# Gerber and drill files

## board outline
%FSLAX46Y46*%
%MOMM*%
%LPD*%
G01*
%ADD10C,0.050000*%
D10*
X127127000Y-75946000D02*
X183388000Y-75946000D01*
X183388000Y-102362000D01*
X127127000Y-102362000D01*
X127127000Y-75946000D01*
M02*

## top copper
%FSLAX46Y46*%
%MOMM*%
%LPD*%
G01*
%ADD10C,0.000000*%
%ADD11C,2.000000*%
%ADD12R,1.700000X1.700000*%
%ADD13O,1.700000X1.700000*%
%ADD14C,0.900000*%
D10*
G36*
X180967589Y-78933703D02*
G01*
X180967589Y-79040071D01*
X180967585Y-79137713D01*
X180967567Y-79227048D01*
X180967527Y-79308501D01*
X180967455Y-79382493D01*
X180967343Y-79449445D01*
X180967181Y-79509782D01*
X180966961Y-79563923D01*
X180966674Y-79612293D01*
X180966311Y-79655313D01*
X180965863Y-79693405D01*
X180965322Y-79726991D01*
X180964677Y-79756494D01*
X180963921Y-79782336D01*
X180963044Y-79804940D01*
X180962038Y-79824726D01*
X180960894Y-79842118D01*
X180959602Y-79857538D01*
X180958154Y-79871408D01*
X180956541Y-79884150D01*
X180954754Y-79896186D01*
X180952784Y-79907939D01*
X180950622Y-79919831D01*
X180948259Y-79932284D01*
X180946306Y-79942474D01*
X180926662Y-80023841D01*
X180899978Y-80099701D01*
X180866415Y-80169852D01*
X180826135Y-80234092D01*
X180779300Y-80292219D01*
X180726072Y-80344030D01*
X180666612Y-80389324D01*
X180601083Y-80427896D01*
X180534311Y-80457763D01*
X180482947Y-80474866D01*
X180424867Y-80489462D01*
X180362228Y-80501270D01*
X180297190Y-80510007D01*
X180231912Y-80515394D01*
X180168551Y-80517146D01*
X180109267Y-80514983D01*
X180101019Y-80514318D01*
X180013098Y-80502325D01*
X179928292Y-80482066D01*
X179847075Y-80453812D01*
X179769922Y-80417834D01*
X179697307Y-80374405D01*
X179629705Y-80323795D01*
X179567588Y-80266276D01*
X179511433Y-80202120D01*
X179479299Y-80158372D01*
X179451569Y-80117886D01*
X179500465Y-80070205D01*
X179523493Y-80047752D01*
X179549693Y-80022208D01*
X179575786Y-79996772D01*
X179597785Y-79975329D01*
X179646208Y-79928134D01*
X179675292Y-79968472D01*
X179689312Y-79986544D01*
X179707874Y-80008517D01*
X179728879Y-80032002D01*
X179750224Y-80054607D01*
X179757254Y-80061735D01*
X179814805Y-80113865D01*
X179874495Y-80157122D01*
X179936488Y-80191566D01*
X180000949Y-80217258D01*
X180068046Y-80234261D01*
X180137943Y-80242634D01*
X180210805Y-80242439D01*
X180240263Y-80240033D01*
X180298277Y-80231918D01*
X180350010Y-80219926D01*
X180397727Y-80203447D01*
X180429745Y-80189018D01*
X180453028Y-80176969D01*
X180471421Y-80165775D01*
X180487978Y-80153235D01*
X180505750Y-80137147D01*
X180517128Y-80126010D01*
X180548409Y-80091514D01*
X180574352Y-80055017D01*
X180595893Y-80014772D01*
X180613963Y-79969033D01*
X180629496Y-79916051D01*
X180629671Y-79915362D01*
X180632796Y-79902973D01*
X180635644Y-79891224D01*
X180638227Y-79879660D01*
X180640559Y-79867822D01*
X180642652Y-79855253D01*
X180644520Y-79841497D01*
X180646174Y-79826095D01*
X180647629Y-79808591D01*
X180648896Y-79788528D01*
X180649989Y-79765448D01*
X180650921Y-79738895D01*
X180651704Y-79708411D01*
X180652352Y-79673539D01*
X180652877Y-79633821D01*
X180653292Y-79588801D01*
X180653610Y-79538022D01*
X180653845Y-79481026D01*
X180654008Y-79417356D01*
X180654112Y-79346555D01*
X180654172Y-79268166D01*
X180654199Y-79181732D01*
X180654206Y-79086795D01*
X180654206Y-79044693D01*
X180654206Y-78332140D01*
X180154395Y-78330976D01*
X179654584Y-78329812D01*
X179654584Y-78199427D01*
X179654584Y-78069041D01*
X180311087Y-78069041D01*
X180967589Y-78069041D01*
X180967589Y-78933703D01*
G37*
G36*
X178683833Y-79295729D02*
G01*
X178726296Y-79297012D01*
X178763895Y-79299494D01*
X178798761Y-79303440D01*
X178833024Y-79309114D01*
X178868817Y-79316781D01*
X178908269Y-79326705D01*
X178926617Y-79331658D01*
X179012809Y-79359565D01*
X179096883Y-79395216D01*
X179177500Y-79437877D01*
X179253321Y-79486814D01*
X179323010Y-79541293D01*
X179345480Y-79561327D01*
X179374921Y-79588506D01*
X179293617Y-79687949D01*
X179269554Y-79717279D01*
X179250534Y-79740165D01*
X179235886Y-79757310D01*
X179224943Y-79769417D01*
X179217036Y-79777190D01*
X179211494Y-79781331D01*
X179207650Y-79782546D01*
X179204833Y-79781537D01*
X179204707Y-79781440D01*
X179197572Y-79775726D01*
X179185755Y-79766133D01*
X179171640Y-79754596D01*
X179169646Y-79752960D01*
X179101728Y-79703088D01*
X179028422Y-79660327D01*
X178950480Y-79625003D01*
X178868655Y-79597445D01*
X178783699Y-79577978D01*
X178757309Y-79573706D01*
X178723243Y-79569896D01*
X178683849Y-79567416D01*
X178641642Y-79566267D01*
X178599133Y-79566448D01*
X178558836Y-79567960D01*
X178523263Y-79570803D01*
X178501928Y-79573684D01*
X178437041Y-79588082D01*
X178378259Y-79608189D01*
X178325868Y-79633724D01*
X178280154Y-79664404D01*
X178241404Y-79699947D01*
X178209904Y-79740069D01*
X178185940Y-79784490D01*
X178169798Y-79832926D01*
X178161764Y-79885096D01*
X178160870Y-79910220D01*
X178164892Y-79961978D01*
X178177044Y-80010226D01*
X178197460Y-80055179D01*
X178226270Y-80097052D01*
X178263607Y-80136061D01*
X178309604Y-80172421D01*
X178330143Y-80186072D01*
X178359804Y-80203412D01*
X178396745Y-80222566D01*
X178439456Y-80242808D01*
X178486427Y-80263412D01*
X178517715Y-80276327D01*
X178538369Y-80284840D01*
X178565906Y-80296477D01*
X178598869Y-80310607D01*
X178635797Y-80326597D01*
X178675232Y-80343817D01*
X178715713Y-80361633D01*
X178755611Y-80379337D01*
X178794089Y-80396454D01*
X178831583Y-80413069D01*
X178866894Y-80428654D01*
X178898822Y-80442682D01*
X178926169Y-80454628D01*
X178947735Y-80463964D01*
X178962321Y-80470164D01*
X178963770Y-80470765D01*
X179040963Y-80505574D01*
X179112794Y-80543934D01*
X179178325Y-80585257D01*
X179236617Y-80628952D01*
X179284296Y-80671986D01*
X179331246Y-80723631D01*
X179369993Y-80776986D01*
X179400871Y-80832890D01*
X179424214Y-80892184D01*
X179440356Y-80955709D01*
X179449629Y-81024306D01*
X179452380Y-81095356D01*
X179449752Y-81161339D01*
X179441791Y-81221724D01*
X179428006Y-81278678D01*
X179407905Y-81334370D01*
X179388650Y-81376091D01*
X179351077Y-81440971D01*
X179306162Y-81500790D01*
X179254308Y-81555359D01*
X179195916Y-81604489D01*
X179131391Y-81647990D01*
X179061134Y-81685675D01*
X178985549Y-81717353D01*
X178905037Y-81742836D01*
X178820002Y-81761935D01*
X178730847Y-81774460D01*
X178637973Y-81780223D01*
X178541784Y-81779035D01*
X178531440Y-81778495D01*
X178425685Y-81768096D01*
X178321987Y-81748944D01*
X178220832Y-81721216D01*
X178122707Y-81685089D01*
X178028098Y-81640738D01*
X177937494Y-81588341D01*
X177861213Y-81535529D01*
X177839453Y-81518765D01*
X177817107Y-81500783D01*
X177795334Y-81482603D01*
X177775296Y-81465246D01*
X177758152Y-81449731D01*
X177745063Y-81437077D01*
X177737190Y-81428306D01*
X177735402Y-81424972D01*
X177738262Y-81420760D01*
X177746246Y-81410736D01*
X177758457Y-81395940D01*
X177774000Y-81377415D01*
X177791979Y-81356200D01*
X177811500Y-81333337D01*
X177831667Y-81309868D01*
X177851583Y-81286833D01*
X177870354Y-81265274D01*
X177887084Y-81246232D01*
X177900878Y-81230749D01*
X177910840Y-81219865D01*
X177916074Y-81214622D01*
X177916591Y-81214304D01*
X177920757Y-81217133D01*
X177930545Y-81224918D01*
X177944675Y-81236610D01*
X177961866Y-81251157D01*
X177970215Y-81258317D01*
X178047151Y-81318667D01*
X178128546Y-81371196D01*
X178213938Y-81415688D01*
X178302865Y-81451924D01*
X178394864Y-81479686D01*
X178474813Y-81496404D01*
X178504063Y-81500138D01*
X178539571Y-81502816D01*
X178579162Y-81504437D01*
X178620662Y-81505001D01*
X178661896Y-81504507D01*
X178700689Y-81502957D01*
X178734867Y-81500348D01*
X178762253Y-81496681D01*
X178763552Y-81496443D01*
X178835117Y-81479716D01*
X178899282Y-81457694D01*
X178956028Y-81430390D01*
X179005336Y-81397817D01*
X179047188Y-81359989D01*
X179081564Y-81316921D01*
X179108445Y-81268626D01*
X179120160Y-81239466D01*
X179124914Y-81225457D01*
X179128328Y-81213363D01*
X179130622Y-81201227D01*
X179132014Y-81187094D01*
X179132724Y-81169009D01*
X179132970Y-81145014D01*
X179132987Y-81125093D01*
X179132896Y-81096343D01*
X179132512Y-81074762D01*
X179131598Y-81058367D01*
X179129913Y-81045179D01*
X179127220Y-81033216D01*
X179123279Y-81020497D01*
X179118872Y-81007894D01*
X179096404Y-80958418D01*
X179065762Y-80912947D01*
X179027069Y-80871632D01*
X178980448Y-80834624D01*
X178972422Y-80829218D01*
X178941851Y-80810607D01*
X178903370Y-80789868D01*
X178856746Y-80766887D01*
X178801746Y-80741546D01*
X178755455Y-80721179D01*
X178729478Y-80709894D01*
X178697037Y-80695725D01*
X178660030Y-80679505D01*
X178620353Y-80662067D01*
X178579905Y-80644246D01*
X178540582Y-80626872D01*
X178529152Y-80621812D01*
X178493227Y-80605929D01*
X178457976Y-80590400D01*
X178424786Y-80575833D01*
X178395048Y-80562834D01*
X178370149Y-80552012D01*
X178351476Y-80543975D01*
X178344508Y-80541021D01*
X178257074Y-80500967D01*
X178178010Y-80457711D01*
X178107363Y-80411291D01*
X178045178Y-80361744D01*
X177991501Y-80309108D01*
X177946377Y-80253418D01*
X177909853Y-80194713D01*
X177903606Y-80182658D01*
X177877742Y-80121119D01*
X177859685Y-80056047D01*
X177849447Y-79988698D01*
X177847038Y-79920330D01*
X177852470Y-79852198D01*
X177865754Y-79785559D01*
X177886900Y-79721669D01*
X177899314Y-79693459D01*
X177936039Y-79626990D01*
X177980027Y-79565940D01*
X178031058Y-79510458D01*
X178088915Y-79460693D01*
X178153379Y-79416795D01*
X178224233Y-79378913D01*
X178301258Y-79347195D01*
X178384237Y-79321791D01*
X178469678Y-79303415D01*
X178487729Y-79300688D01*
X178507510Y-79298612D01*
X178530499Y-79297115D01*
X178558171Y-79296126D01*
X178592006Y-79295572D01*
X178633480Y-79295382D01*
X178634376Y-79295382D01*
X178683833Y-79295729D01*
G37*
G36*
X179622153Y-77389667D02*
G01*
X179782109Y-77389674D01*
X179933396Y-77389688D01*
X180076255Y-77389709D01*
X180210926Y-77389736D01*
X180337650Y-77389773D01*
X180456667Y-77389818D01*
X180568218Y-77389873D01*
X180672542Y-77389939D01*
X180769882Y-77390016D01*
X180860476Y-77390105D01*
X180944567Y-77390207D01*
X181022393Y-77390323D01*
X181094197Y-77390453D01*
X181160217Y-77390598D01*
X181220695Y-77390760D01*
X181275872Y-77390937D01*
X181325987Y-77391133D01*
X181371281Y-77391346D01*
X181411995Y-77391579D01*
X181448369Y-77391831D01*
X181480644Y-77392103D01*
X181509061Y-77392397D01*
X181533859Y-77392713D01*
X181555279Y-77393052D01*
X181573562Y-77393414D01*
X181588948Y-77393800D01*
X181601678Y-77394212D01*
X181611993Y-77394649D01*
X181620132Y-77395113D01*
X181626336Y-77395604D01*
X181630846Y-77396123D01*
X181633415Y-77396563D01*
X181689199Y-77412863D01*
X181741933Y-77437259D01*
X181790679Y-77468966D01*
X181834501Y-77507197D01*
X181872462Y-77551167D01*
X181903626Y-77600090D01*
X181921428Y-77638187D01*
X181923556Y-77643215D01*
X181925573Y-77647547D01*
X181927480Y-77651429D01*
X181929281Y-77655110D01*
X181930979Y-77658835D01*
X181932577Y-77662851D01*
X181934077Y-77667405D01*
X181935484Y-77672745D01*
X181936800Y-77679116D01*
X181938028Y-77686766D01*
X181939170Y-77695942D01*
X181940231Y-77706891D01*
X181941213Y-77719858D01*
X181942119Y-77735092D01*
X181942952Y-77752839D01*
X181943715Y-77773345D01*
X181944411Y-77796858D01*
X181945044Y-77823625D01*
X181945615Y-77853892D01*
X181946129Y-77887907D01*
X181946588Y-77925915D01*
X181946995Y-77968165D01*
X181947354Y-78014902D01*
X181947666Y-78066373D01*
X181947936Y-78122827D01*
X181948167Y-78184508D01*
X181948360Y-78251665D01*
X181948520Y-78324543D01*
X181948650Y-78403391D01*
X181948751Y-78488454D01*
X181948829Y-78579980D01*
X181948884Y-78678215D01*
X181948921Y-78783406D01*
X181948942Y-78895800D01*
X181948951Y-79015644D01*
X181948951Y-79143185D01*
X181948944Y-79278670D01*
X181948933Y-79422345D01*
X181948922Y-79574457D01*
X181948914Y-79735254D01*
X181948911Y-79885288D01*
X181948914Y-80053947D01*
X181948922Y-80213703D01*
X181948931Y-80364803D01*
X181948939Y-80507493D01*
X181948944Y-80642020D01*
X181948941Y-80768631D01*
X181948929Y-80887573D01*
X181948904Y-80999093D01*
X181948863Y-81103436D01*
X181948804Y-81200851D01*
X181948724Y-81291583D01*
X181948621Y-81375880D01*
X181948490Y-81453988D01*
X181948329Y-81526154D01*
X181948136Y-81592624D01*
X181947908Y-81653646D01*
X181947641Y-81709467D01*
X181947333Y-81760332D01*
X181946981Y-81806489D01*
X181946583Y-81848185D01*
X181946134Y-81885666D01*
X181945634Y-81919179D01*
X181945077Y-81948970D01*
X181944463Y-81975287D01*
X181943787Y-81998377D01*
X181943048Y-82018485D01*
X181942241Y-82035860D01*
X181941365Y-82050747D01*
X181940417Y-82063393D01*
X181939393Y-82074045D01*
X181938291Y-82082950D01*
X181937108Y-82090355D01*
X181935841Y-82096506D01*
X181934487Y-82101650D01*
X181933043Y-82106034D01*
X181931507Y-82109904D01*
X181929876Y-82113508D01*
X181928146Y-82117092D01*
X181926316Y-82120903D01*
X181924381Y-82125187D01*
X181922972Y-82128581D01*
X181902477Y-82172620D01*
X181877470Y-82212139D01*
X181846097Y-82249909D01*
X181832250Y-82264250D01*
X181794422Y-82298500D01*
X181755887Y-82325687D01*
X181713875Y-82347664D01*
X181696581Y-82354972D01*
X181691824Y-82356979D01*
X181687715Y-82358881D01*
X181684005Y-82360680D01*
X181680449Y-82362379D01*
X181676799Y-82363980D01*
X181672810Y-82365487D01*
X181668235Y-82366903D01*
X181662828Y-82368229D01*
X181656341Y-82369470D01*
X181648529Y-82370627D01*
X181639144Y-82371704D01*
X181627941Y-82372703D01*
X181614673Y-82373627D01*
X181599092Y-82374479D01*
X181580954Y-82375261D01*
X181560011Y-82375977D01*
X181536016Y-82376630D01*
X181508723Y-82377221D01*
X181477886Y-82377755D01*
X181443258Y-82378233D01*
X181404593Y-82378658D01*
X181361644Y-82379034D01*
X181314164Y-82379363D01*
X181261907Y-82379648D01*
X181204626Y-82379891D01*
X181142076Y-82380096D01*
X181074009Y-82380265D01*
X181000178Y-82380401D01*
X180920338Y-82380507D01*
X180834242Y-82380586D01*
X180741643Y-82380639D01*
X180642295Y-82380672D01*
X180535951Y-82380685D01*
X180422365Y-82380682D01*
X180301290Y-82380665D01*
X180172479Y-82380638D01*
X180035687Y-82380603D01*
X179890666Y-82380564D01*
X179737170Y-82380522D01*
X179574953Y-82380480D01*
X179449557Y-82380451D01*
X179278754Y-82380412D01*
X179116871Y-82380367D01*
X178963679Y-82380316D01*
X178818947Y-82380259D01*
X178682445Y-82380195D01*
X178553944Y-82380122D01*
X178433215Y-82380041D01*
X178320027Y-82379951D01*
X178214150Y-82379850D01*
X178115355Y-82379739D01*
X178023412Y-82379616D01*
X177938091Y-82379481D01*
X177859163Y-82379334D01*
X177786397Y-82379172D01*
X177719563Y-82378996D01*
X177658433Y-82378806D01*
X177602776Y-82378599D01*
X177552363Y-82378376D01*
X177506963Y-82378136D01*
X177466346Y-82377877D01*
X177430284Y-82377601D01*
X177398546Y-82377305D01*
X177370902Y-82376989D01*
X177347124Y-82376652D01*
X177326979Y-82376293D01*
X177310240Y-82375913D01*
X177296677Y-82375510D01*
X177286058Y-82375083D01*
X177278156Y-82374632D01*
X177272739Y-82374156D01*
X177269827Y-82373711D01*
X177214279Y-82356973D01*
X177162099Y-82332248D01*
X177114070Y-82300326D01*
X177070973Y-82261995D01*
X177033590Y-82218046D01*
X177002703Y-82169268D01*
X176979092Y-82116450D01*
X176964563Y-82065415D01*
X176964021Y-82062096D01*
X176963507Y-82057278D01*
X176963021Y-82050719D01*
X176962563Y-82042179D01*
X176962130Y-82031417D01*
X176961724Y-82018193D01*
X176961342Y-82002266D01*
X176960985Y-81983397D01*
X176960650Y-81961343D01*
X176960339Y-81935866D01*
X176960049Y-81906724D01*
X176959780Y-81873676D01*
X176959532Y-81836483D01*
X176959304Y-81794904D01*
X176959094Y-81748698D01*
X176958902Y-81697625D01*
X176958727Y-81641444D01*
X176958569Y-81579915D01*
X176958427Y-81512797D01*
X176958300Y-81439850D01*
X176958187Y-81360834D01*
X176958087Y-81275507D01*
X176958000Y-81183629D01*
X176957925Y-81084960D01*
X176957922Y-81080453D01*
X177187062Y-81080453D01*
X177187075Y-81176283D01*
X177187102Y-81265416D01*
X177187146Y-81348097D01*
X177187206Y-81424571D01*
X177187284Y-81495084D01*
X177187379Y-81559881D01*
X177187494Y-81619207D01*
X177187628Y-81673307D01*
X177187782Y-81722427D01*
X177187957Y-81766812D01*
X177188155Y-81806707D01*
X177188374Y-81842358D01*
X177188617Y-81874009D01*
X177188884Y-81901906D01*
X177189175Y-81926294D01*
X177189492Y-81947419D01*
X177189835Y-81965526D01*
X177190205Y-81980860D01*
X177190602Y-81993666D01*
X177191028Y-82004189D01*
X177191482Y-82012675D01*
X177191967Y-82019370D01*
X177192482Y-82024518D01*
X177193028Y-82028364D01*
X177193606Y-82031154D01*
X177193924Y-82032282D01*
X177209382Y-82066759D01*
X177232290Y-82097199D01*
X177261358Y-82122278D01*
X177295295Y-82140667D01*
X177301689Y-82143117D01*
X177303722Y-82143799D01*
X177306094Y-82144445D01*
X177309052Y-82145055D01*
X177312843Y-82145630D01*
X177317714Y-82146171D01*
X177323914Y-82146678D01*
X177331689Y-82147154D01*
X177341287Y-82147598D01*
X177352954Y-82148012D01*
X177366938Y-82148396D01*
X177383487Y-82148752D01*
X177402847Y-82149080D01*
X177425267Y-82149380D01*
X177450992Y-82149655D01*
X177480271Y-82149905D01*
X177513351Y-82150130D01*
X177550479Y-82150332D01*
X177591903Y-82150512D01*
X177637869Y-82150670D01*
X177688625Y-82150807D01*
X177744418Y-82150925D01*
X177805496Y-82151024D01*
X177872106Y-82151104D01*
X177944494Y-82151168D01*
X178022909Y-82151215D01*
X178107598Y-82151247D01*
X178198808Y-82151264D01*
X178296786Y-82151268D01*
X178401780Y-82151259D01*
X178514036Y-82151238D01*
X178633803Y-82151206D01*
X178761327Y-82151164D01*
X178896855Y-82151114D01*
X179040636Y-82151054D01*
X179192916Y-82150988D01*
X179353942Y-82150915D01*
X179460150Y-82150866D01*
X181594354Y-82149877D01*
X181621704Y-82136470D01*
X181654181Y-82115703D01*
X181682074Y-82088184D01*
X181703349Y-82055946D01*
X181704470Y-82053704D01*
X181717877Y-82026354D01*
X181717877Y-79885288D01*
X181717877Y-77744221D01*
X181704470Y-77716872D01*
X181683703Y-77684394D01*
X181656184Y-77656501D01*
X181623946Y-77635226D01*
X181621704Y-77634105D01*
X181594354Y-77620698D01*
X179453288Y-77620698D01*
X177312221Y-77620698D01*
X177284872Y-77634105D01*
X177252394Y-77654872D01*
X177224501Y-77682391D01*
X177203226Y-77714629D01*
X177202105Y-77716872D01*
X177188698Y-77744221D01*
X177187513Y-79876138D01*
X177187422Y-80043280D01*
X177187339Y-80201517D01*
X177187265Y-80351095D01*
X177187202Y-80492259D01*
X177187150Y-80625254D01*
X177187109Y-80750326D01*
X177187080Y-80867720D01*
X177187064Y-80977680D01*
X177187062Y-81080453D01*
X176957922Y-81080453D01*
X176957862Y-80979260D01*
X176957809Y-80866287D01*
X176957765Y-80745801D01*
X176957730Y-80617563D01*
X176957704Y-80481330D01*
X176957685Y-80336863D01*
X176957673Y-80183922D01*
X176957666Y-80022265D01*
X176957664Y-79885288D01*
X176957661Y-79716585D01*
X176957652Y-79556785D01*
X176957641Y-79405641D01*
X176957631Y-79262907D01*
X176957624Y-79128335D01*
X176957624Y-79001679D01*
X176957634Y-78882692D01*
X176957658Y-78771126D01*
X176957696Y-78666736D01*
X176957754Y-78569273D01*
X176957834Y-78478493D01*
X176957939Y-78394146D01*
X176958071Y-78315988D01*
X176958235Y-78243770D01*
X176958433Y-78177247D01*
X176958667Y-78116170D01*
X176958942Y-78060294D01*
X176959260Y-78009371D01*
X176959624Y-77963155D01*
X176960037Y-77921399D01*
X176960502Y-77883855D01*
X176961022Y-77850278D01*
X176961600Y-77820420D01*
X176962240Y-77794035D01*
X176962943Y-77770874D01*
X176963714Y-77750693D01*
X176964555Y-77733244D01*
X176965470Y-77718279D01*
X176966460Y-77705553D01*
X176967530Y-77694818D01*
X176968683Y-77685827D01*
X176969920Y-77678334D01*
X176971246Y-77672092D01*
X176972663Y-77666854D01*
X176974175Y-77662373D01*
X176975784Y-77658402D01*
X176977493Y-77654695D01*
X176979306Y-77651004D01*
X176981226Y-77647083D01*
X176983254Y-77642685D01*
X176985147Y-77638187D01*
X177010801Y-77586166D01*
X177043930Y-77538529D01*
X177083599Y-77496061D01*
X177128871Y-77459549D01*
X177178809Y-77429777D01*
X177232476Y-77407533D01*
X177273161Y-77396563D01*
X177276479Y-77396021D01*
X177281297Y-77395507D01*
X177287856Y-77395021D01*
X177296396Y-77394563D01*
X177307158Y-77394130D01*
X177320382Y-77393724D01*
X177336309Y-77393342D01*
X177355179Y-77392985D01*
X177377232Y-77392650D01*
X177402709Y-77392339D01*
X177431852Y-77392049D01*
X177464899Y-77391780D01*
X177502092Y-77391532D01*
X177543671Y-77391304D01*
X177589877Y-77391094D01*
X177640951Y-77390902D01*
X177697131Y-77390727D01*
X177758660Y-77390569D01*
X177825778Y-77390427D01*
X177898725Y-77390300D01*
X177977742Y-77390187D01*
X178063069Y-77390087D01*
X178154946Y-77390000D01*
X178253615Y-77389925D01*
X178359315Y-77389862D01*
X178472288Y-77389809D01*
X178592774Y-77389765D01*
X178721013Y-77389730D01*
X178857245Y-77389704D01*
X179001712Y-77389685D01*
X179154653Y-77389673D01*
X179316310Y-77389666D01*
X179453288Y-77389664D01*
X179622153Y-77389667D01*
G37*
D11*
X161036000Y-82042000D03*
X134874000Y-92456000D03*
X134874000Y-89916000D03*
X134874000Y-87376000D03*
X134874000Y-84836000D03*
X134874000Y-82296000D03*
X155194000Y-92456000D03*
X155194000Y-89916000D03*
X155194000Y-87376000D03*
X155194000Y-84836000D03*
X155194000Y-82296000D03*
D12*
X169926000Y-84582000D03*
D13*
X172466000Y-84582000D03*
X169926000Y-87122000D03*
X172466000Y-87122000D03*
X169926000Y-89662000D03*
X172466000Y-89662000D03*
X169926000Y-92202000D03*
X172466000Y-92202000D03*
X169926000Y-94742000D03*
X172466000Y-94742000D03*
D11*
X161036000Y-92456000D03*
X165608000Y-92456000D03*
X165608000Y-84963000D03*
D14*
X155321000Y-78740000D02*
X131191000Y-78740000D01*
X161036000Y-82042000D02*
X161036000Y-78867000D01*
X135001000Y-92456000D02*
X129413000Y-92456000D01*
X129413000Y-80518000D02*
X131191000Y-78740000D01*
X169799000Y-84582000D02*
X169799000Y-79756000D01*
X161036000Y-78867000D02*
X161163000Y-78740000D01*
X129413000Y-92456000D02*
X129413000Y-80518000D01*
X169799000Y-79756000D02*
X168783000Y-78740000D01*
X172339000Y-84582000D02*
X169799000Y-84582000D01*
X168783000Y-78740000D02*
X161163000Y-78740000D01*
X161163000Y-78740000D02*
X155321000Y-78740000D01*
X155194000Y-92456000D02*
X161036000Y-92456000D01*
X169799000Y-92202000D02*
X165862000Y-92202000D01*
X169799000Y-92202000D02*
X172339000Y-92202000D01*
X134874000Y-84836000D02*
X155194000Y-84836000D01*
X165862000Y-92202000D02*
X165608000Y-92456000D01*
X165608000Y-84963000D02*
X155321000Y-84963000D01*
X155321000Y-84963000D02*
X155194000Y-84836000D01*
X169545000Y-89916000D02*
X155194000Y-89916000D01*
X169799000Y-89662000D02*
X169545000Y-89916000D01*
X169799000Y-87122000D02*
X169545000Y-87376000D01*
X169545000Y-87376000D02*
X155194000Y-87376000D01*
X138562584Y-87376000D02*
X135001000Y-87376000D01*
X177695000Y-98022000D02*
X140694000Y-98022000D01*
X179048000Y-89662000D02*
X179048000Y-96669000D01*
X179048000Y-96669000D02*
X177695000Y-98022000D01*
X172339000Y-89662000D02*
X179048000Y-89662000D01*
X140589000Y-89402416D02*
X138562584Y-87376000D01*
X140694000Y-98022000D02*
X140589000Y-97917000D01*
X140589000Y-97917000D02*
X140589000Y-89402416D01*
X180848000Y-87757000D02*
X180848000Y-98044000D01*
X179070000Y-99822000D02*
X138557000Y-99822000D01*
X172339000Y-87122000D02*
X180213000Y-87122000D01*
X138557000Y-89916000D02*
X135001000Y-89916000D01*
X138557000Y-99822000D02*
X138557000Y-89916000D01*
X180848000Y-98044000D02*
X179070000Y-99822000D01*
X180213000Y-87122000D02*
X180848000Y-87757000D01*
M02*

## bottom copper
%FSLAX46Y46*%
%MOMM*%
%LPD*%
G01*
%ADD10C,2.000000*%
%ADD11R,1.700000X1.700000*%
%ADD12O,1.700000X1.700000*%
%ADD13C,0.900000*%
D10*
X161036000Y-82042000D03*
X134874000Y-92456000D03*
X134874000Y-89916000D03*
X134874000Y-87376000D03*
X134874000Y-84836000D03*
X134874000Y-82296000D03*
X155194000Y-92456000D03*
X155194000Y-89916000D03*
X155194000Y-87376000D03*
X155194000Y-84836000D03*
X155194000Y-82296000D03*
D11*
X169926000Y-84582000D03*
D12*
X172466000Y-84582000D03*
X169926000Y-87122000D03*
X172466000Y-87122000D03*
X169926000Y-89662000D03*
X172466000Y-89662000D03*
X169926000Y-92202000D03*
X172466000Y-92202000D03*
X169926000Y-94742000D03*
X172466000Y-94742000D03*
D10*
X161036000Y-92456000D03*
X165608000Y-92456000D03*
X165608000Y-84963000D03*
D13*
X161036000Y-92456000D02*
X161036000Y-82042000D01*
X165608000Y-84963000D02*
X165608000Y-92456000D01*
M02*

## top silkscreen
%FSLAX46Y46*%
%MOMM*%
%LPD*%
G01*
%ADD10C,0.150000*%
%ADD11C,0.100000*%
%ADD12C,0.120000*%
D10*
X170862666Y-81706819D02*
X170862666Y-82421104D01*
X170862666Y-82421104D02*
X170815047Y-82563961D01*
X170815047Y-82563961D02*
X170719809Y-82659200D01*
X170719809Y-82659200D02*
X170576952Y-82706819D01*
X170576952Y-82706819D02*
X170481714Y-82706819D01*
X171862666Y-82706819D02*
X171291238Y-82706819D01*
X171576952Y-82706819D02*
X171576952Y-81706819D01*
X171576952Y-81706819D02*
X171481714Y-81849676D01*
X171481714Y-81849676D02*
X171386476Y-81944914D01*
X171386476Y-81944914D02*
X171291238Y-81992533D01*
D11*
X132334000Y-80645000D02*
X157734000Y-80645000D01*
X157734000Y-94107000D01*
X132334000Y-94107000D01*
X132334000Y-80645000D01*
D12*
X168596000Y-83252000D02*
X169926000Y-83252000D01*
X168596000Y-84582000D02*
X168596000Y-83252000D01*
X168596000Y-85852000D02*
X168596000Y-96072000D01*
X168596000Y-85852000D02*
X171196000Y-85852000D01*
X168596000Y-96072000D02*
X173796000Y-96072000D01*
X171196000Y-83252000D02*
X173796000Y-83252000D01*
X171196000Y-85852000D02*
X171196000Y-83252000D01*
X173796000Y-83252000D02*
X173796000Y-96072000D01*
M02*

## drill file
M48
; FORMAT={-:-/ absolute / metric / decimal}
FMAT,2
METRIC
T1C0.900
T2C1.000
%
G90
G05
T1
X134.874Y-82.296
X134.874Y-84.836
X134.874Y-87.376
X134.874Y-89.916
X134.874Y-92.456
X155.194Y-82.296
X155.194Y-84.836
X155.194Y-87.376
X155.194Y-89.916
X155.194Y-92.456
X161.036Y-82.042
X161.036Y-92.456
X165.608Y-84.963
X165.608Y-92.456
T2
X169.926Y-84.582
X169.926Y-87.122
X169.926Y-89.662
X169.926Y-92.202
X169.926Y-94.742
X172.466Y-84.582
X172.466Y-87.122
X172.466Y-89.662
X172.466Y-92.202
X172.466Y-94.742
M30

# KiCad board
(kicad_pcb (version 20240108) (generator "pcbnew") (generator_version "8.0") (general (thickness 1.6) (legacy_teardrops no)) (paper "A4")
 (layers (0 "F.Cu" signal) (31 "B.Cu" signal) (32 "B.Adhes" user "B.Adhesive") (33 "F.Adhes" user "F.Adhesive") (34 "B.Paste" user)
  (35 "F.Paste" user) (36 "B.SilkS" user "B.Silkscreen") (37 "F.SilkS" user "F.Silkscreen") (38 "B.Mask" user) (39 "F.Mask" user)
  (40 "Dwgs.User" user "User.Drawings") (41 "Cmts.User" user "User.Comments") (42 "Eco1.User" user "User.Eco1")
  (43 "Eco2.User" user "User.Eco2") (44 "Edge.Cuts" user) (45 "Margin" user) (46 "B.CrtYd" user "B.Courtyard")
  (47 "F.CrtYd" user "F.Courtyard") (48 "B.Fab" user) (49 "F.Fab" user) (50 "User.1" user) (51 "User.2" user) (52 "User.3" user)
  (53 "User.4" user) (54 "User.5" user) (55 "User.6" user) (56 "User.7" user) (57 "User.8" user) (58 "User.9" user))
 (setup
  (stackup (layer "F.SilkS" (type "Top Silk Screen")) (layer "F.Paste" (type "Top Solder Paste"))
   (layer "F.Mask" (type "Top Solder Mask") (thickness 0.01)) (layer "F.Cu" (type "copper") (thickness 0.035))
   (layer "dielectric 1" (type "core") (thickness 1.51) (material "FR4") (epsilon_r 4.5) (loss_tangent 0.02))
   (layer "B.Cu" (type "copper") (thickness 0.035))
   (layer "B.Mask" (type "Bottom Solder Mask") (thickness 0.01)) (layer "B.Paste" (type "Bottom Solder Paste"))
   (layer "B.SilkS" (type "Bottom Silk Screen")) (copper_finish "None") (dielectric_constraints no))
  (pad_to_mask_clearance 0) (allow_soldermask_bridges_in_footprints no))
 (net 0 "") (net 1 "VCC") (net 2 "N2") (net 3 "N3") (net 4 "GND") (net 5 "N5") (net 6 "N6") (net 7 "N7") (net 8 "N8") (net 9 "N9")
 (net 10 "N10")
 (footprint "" (layer "F.Cu") (at 161.036 82.042)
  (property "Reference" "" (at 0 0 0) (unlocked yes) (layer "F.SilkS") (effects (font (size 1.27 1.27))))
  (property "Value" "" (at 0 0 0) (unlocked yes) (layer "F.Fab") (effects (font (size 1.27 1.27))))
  (pad "6" thru_hole circle (at 0 0) (size 2 2) (drill 0.9) (layers "*.Cu" "*.Mask") (remove_unused_layers no) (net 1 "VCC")))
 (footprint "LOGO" (layer "F.Cu") (at 179.451 79.883)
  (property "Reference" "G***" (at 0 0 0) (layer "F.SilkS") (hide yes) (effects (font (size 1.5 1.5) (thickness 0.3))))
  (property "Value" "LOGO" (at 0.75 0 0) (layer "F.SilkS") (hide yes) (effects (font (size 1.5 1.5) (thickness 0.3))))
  (fp_poly
   (pts (xy 1.516589 -0.949297) (xy 1.516589 -0.842929) (xy 1.516585 -0.745287) (xy 1.516567 -0.655952) (xy 1.516527 -0.574499)
    (xy 1.516455 -0.500507) (xy 1.516343 -0.433555) (xy 1.516181 -0.373218) (xy 1.515961 -0.319077) (xy 1.515674 -0.270707)
    (xy 1.515311 -0.227687) (xy 1.514863 -0.189595) (xy 1.514322 -0.156009) (xy 1.513677 -0.126506) (xy 1.512921 -0.100664)
    (xy 1.512044 -0.07806) (xy 1.511038 -0.058274) (xy 1.509894 -0.040882) (xy 1.508602 -0.025462) (xy 1.507154 -0.011592)
    (xy 1.505541 0.00115) (xy 1.503754 0.013186) (xy 1.501784 0.024939) (xy 1.499622 0.036831) (xy 1.497259 0.049284) (xy 1.495306 0.059474)
    (xy 1.475662 0.140841) (xy 1.448978 0.216701) (xy 1.415415 0.286852) (xy 1.375135 0.351092) (xy 1.3283 0.409219) (xy 1.275072 0.46103)
    (xy 1.215612 0.506324) (xy 1.150083 0.544896) (xy 1.083311 0.574763) (xy 1.031947 0.591866) (xy 0.973867 0.606462) (xy 0.911228 0.61827)
    (xy 0.84619 0.627007) (xy 0.780912 0.632394) (xy 0.717551 0.634146) (xy 0.658267 0.631983) (xy 0.650019 0.631318) (xy 0.562098 0.619325)
    (xy 0.477292 0.599066) (xy 0.396075 0.570812) (xy 0.318922 0.534834) (xy 0.246307 0.491405) (xy 0.178705 0.440795)
    (xy 0.116588 0.383276) (xy 0.060433 0.31912) (xy 0.028299 0.275372) (xy 0.000569 0.234886) (xy 0.049465 0.187205) (xy 0.072493 0.164752)
    (xy 0.098693 0.139208) (xy 0.124786 0.113772) (xy 0.146785 0.092329) (xy 0.195208 0.045134) (xy 0.224292 0.085472)
    (xy 0.238312 0.103544) (xy 0.256874 0.125517) (xy 0.277879 0.149002) (xy 0.299224 0.171607) (xy 0.306254 0.178735)
    (xy 0.363805 0.230865) (xy 0.423495 0.274122) (xy 0.485488 0.308566) (xy 0.549949 0.334258) (xy 0.617046 0.351261)
    (xy 0.686943 0.359634) (xy 0.759805 0.359439) (xy 0.789263 0.357033) (xy 0.847277 0.348918) (xy 0.89901 0.336926) (xy 0.946727 0.320447)
    (xy 0.978745 0.306018) (xy 1.002028 0.293969) (xy 1.020421 0.282775) (xy 1.036978 0.270235) (xy 1.05475 0.254147) (xy 1.066128 0.24301)
    (xy 1.097409 0.208514) (xy 1.123352 0.172017) (xy 1.144893 0.131772) (xy 1.162963 0.086033) (xy 1.178496 0.033051)
    (xy 1.178671 0.032362) (xy 1.181796 0.019973) (xy 1.184644 0.008224) (xy 1.187227 -0.00334) (xy 1.189559 -0.015178)
    (xy 1.191652 -0.027747) (xy 1.19352 -0.041503) (xy 1.195174 -0.056905) (xy 1.196629 -0.074409) (xy 1.197896 -0.094472)
    (xy 1.198989 -0.117552) (xy 1.199921 -0.144105) (xy 1.200704 -0.174589) (xy 1.201352 -0.209461) (xy 1.201877 -0.249179)
    (xy 1.202292 -0.294199) (xy 1.20261 -0.344978) (xy 1.202845 -0.401974) (xy 1.203008 -0.465644) (xy 1.203112 -0.536445)
    (xy 1.203172 -0.614834) (xy 1.203199 -0.701268) (xy 1.203206 -0.796205) (xy 1.203206 -0.838307) (xy 1.203206 -1.55086)
    (xy 0.703395 -1.552024) (xy 0.203584 -1.553188) (xy 0.203584 -1.683573) (xy 0.203584 -1.813959) (xy 0.860087 -1.813959)
    (xy 1.516589 -1.813959))
   (stroke (width 0) (type solid)) (fill solid) (layer "F.Cu"))
  (fp_poly
   (pts (xy -0.767167 -0.587271) (xy -0.724704 -0.585988) (xy -0.687105 -0.583506) (xy -0.652239 -0.57956) (xy -0.617976 -0.573886)
    (xy -0.582183 -0.566219) (xy -0.542731 -0.556295) (xy -0.524383 -0.551342) (xy -0.438191 -0.523435) (xy -0.354117 -0.487784)
    (xy -0.2735 -0.445123) (xy -0.197679 -0.396186) (xy -0.12799 -0.341707) (xy -0.10552 -0.321673) (xy -0.076079 -0.294494)
    (xy -0.157383 -0.195051) (xy -0.181446 -0.165721) (xy -0.200466 -0.142835) (xy -0.215114 -0.12569) (xy -0.226057 -0.113583)
    (xy -0.233964 -0.10581) (xy -0.239506 -0.101669) (xy -0.24335 -0.100454) (xy -0.246167 -0.101463) (xy -0.246293 -0.10156)
    (xy -0.253428 -0.107274) (xy -0.265245 -0.116867) (xy -0.27936 -0.128404) (xy -0.281354 -0.13004) (xy -0.349272 -0.179912)
    (xy -0.422578 -0.222673) (xy -0.50052 -0.257997) (xy -0.582345 -0.285555) (xy -0.667301 -0.305022) (xy -0.693691 -0.309294)
    (xy -0.727757 -0.313104) (xy -0.767151 -0.315584) (xy -0.809358 -0.316733) (xy -0.851867 -0.316552) (xy -0.892164 -0.31504)
    (xy -0.927737 -0.312197) (xy -0.949072 -0.309316) (xy -1.013959 -0.294918) (xy -1.072741 -0.274811) (xy -1.125132 -0.249276)
    (xy -1.170846 -0.218596) (xy -1.209596 -0.183053) (xy -1.241096 -0.142931) (xy -1.26506 -0.09851) (xy -1.281202 -0.050074)
    (xy -1.289236 0.002096) (xy -1.29013 0.02722) (xy -1.286108 0.078978) (xy -1.273956 0.127226) (xy -1.25354 0.172179)
    (xy -1.22473 0.214052) (xy -1.187393 0.253061) (xy -1.141396 0.289421) (xy -1.120857 0.303072) (xy -1.091196 0.320412)
    (xy -1.054255 0.339566) (xy -1.011544 0.359808) (xy -0.964573 0.380412) (xy -0.933285 0.393327) (xy -0.912631 0.40184)
    (xy -0.885094 0.413477) (xy -0.852131 0.427607) (xy -0.815203 0.443597) (xy -0.775768 0.460817) (xy -0.735287 0.478633)
    (xy -0.695389 0.496337) (xy -0.656911 0.513454) (xy -0.619417 0.530069) (xy -0.584106 0.545654) (xy -0.552178 0.559682)
    (xy -0.524831 0.571628) (xy -0.503265 0.580964) (xy -0.488679 0.587164) (xy -0.48723 0.587765) (xy -0.410037 0.622574)
    (xy -0.338206 0.660934) (xy -0.272675 0.702257) (xy -0.214383 0.745952) (xy -0.166704 0.788986) (xy -0.119754 0.840631)
    (xy -0.081007 0.893986) (xy -0.050129 0.94989) (xy -0.026786 1.009184) (xy -0.010644 1.072709) (xy -0.001371 1.141306)
    (xy 0.00138 1.212356) (xy -0.001248 1.278339) (xy -0.009209 1.338724) (xy -0.022994 1.395678) (xy -0.043095 1.45137)
    (xy -0.06235 1.493091) (xy -0.099923 1.557971) (xy -0.144838 1.61779) (xy -0.196692 1.672359) (xy -0.255084 1.721489)
    (xy -0.319609 1.76499) (xy -0.389866 1.802675) (xy -0.465451 1.834353) (xy -0.545963 1.859836) (xy -0.630998 1.878935)
    (xy -0.720153 1.89146) (xy -0.813027 1.897223) (xy -0.909216 1.896035) (xy -0.91956 1.895495) (xy -1.025315 1.885096)
    (xy -1.129013 1.865944) (xy -1.230168 1.838216) (xy -1.328293 1.802089) (xy -1.422902 1.757738) (xy -1.513506 1.705341)
    (xy -1.589787 1.652529) (xy -1.611547 1.635765) (xy -1.633893 1.617783) (xy -1.655666 1.599603) (xy -1.675704 1.582246)
    (xy -1.692848 1.566731) (xy -1.705937 1.554077) (xy -1.71381 1.545306) (xy -1.715598 1.541972) (xy -1.712738 1.53776)
    (xy -1.704754 1.527736) (xy -1.692543 1.51294) (xy -1.677 1.494415) (xy -1.659021 1.4732) (xy -1.6395 1.450337) (xy -1.619333 1.426868)
    (xy -1.599417 1.403833) (xy -1.580646 1.382274) (xy -1.563916 1.363232) (xy -1.550122 1.347749) (xy -1.54016 1.336865)
    (xy -1.534926 1.331622) (xy -1.534409 1.331304) (xy -1.530243 1.334133) (xy -1.520455 1.341918) (xy -1.506325 1.35361)
    (xy -1.489134 1.368157) (xy -1.480785 1.375317) (xy -1.403849 1.435667) (xy -1.322454 1.488196) (xy -1.237062 1.532688)
    (xy -1.148135 1.568924) (xy -1.056136 1.596686) (xy -0.976187 1.613404) (xy -0.946937 1.617138) (xy -0.911429 1.619816)
    (xy -0.871838 1.621437) (xy -0.830338 1.622001) (xy -0.789104 1.621507) (xy -0.750311 1.619957) (xy -0.716133 1.617348)
    (xy -0.688747 1.613681) (xy -0.687448 1.613443) (xy -0.615883 1.596716) (xy -0.551718 1.574694) (xy -0.494972 1.54739)
    (xy -0.445664 1.514817) (xy -0.403812 1.476989) (xy -0.369436 1.433921) (xy -0.342555 1.385626) (xy -0.33084 1.356466)
    (xy -0.326086 1.342457) (xy -0.322672 1.330363) (xy -0.320378 1.318227) (xy -0.318986 1.304094) (xy -0.318276 1.286009)
    (xy -0.31803 1.262014) (xy -0.318013 1.242093) (xy -0.318104 1.213343) (xy -0.318488 1.191762) (xy -0.319402 1.175367)
    (xy -0.321087 1.162179) (xy -0.32378 1.150216) (xy -0.327721 1.137497) (xy -0.332128 1.124894) (xy -0.354596 1.075418)
    (xy -0.385238 1.029947) (xy -0.423931 0.988632) (xy -0.470552 0.951624) (xy -0.478578 0.946218) (xy -0.509149 0.927607)
    (xy -0.54763 0.906868) (xy -0.594254 0.883887) (xy -0.649254 0.858546) (xy -0.695545 0.838179) (xy -0.721522 0.826894)
    (xy -0.753963 0.812725) (xy -0.79097 0.796505) (xy -0.830647 0.779067) (xy -0.871095 0.761246) (xy -0.910418 0.743872)
    (xy -0.921848 0.738812) (xy -0.957773 0.722929) (xy -0.993024 0.7074) (xy -1.026214 0.692833) (xy -1.055952 0.679834)
    (xy -1.080851 0.669012) (xy -1.099524 0.660975) (xy -1.106492 0.658021) (xy -1.193926 0.617967) (xy -1.27299 0.574711)
    (xy -1.343637 0.528291) (xy -1.405822 0.478744) (xy -1.459499 0.426108) (xy -1.504623 0.370418) (xy -1.541147 0.311713)
    (xy -1.547394 0.299658) (xy -1.573258 0.238119) (xy -1.591315 0.173047) (xy -1.601553 0.105698) (xy -1.603962 0.03733)
    (xy -1.59853 -0.030802) (xy -1.585246 -0.097441) (xy -1.5641 -0.161331) (xy -1.551686 -0.189541) (xy -1.514961 -0.25601)
    (xy -1.470973 -0.31706) (xy -1.419942 -0.372542) (xy -1.362085 -0.422307) (xy -1.297621 -0.466205) (xy -1.226767 -0.504087)
    (xy -1.149742 -0.535805) (xy -1.066763 -0.561209) (xy -0.981322 -0.579585) (xy -0.963271 -0.582312) (xy -0.94349 -0.584388)
    (xy -0.920501 -0.585885) (xy -0.892829 -0.586874) (xy -0.858994 -0.587428) (xy -0.81752 -0.587618) (xy -0.816624 -0.587618))
   (stroke (width 0) (type solid)) (fill solid) (layer "F.Cu"))
  (fp_poly
   (pts (xy 0.171153 -2.493333) (xy 0.331109 -2.493326) (xy 0.482396 -2.493312) (xy 0.625255 -2.493291) (xy 0.759926 -2.493264)
    (xy 0.88665 -2.493227) (xy 1.005667 -2.493182) (xy 1.117218 -2.493127) (xy 1.221542 -2.493061) (xy 1.318882 -2.492984)
    (xy 1.409476 -2.492895) (xy 1.493567 -2.492793) (xy 1.571393 -2.492677) (xy 1.643197 -2.492547) (xy 1.709217 -2.492402)
    (xy 1.769695 -2.49224) (xy 1.824872 -2.492063) (xy 1.874987 -2.491867) (xy 1.920281 -2.491654) (xy 1.960995 -2.491421)
    (xy 1.997369 -2.491169) (xy 2.029644 -2.490897) (xy 2.058061 -2.490603) (xy 2.082859 -2.490287) (xy 2.104279 -2.489948)
    (xy 2.122562 -2.489586) (xy 2.137948 -2.4892) (xy 2.150678 -2.488788) (xy 2.160993 -2.488351) (xy 2.169132 -2.487887)
    (xy 2.175336 -2.487396) (xy 2.179846 -2.486877) (xy 2.182415 -2.486437) (xy 2.238199 -2.470137) (xy 2.290933 -2.445741)
    (xy 2.339679 -2.414034) (xy 2.383501 -2.375803) (xy 2.421462 -2.331833) (xy 2.452626 -2.28291) (xy 2.470428 -2.244813)
    (xy 2.472556 -2.239785) (xy 2.474573 -2.235453) (xy 2.47648 -2.231571) (xy 2.478281 -2.22789) (xy 2.479979 -2.224165)
    (xy 2.481577 -2.220149) (xy 2.483077 -2.215595) (xy 2.484484 -2.210255) (xy 2.4858 -2.203884) (xy 2.487028 -2.196234)
    (xy 2.48817 -2.187058) (xy 2.489231 -2.176109) (xy 2.490213 -2.163142) (xy 2.491119 -2.147908) (xy 2.491952 -2.130161)
    (xy 2.492715 -2.109655) (xy 2.493411 -2.086142) (xy 2.494044 -2.059375) (xy 2.494615 -2.029108) (xy 2.495129 -1.995093)
    (xy 2.495588 -1.957085) (xy 2.495995 -1.914835) (xy 2.496354 -1.868098) (xy 2.496666 -1.816627) (xy 2.496936 -1.760173)
    (xy 2.497167 -1.698492) (xy 2.49736 -1.631335) (xy 2.49752 -1.558457) (xy 2.49765 -1.479609) (xy 2.497751 -1.394546)
    (xy 2.497829 -1.30302) (xy 2.497884 -1.204785) (xy 2.497921 -1.099594) (xy 2.497942 -0.9872) (xy 2.497951 -0.867356)
    (xy 2.497951 -0.739815) (xy 2.497944 -0.60433) (xy 2.497933 -0.460655) (xy 2.497922 -0.308543) (xy 2.497914 -0.147746)
    (xy 2.497911 0.002288) (xy 2.497914 0.170947) (xy 2.497922 0.330703) (xy 2.497931 0.481803) (xy 2.497939 0.624493) (xy 2.497944 0.75902)
    (xy 2.497941 0.885631) (xy 2.497929 1.004573) (xy 2.497904 1.116093) (xy 2.497863 1.220436) (xy 2.497804 1.317851)
    (xy 2.497724 1.408583) (xy 2.497621 1.49288) (xy 2.49749 1.570988) (xy 2.497329 1.643154) (xy 2.497136 1.709624) (xy 2.496908 1.770646)
    (xy 2.496641 1.826467) (xy 2.496333 1.877332) (xy 2.495981 1.923489) (xy 2.495583 1.965185) (xy 2.495134 2.002666)
    (xy 2.494634 2.036179) (xy 2.494077 2.06597) (xy 2.493463 2.092287) (xy 2.492787 2.115377) (xy 2.492048 2.135485) (xy 2.491241 2.15286)
    (xy 2.490365 2.167747) (xy 2.489417 2.180393) (xy 2.488393 2.191045) (xy 2.487291 2.19995) (xy 2.486108 2.207355) (xy 2.484841 2.213506)
    (xy 2.483487 2.21865) (xy 2.482043 2.223034) (xy 2.480507 2.226904) (xy 2.478876 2.230508) (xy 2.477146 2.234092) (xy 2.475316 2.237903)
    (xy 2.473381 2.242187) (xy 2.471972 2.245581) (xy 2.451477 2.28962) (xy 2.42647 2.329139) (xy 2.395097 2.366909) (xy 2.38125 2.38125)
    (xy 2.343422 2.4155) (xy 2.304887 2.442687) (xy 2.262875 2.464664) (xy 2.245581 2.471972) (xy 2.240824 2.473979) (xy 2.236715 2.475881)
    (xy 2.233005 2.47768) (xy 2.229449 2.479379) (xy 2.225799 2.48098) (xy 2.22181 2.482487) (xy 2.217235 2.483903) (xy 2.211828 2.485229)
    (xy 2.205341 2.48647) (xy 2.197529 2.487627) (xy 2.188144 2.488704) (xy 2.176941 2.489703) (xy 2.163673 2.490627) (xy 2.148092 2.491479)
    (xy 2.129954 2.492261) (xy 2.109011 2.492977) (xy 2.085016 2.49363) (xy 2.057723 2.494221) (xy 2.026886 2.494755) (xy 1.992258 2.495233)
    (xy 1.953593 2.495658) (xy 1.910644 2.496034) (xy 1.863164 2.496363) (xy 1.810907 2.496648) (xy 1.753626 2.496891)
    (xy 1.691076 2.497096) (xy 1.623009 2.497265) (xy 1.549178 2.497401) (xy 1.469338 2.497507) (xy 1.383242 2.497586)
    (xy 1.290643 2.497639) (xy 1.191295 2.497672) (xy 1.084951 2.497685) (xy 0.971365 2.497682) (xy 0.85029 2.497665) (xy 0.721479 2.497638)
    (xy 0.584687 2.497603) (xy 0.439666 2.497564) (xy 0.28617 2.497522) (xy 0.123953 2.49748) (xy -0.001443 2.497451)
    (xy -0.172246 2.497412) (xy -0.334129 2.497367) (xy -0.487321 2.497316) (xy -0.632053 2.497259) (xy -0.768555 2.497195)
    (xy -0.897056 2.497122) (xy -1.017785 2.497041) (xy -1.130973 2.496951) (xy -1.23685 2.49685) (xy -1.335645 2.496739)
    (xy -1.427588 2.496616) (xy -1.512909 2.496481) (xy -1.591837 2.496334) (xy -1.664603 2.496172) (xy -1.731437 2.495996)
    (xy -1.792567 2.495806) (xy -1.848224 2.495599) (xy -1.898637 2.495376) (xy -1.944037 2.495136) (xy -1.984654 2.494877)
    (xy -2.020716 2.494601) (xy -2.052454 2.494305) (xy -2.080098 2.493989) (xy -2.103876 2.493652) (xy -2.124021 2.493293)
    (xy -2.14076 2.492913) (xy -2.154323 2.49251) (xy -2.164942 2.492083) (xy -2.172844 2.491632) (xy -2.178261 2.491156)
    (xy -2.181173 2.490711) (xy -2.236721 2.473973) (xy -2.288901 2.449248) (xy -2.33693 2.417326) (xy -2.380027 2.378995)
    (xy -2.41741 2.335046) (xy -2.448297 2.286268) (xy -2.471908 2.23345) (xy -2.486437 2.182415) (xy -2.486979 2.179096)
    (xy -2.487493 2.174278) (xy -2.487979 2.167719) (xy -2.488437 2.159179) (xy -2.48887 2.148417) (xy -2.489276 2.135193)
    (xy -2.489658 2.119266) (xy -2.490015 2.100397) (xy -2.49035 2.078343) (xy -2.490661 2.052866) (xy -2.490951 2.023724)
    (xy -2.49122 1.990676) (xy -2.491468 1.953483) (xy -2.491696 1.911904) (xy -2.491906 1.865698) (xy -2.492098 1.814625)
    (xy -2.492273 1.758444) (xy -2.492431 1.696915) (xy -2.492573 1.629797) (xy -2.4927 1.55685) (xy -2.492813 1.477834)
    (xy -2.492913 1.392507) (xy -2.493 1.300629) (xy -2.493075 1.20196) (xy -2.493078 1.197453) (xy -2.263938 1.197453)
    (xy -2.263925 1.293283) (xy -2.263898 1.382416) (xy -2.263854 1.465097) (xy -2.263794 1.541571) (xy -2.263716 1.612084)
    (xy -2.263621 1.676881) (xy -2.263506 1.736207) (xy -2.263372 1.790307) (xy -2.263218 1.839427) (xy -2.263043 1.883812)
    (xy -2.262845 1.923707) (xy -2.262626 1.959358) (xy -2.262383 1.991009) (xy -2.262116 2.018906) (xy -2.261825 2.043294)
    (xy -2.261508 2.064419) (xy -2.261165 2.082526) (xy -2.260795 2.09786) (xy -2.260398 2.110666) (xy -2.259972 2.121189)
    (xy -2.259518 2.129675) (xy -2.259033 2.13637) (xy -2.258518 2.141518) (xy -2.257972 2.145364) (xy -2.257394 2.148154)
    (xy -2.257076 2.149282) (xy -2.241618 2.183759) (xy -2.21871 2.214199) (xy -2.189642 2.239278) (xy -2.155705 2.257667)
    (xy -2.149311 2.260117) (xy -2.147278 2.260799) (xy -2.144906 2.261445) (xy -2.141948 2.262055) (xy -2.138157 2.26263)
    (xy -2.133286 2.263171) (xy -2.127086 2.263678) (xy -2.119311 2.264154) (xy -2.109713 2.264598) (xy -2.098046 2.265012)
    (xy -2.084062 2.265396) (xy -2.067513 2.265752) (xy -2.048153 2.26608) (xy -2.025733 2.26638) (xy -2.000008 2.266655)
    (xy -1.970729 2.266905) (xy -1.937649 2.26713) (xy -1.900521 2.267332) (xy -1.859097 2.267512) (xy -1.813131 2.26767)
    (xy -1.762375 2.267807) (xy -1.706582 2.267925) (xy -1.645504 2.268024) (xy -1.578894 2.268104) (xy -1.506506 2.268168)
    (xy -1.428091 2.268215) (xy -1.343402 2.268247) (xy -1.252192 2.268264) (xy -1.154214 2.268268) (xy -1.04922 2.268259)
    (xy -0.936964 2.268238) (xy -0.817197 2.268206) (xy -0.689673 2.268164) (xy -0.554145 2.268114) (xy -0.410364 2.268054)
    (xy -0.258084 2.267988) (xy -0.097058 2.267915) (xy 0.00915 2.267866) (xy 2.143354 2.266877) (xy 2.170704 2.25347)
    (xy 2.203181 2.232703) (xy 2.231074 2.205184) (xy 2.252349 2.172946) (xy 2.25347 2.170704) (xy 2.266877 2.143354) (xy 2.266877 0.002288)
    (xy 2.266877 -2.138779) (xy 2.25347 -2.166128) (xy 2.232703 -2.198606) (xy 2.205184 -2.226499) (xy 2.172946 -2.247774)
    (xy 2.170704 -2.248895) (xy 2.143354 -2.262302) (xy 0.002288 -2.262302) (xy -2.138779 -2.262302) (xy -2.166128 -2.248895)
    (xy -2.198606 -2.228128) (xy -2.226499 -2.200609) (xy -2.247774 -2.168371) (xy -2.248895 -2.166128) (xy -2.262302 -2.138779)
    (xy -2.263487 -0.006862) (xy -2.263578 0.16028) (xy -2.263661 0.318517) (xy -2.263735 0.468095) (xy -2.263798 0.609259)
    (xy -2.26385 0.742254) (xy -2.263891 0.867326) (xy -2.26392 0.98472) (xy -2.263936 1.09468) (xy -2.263938 1.197453)
    (xy -2.493078 1.197453) (xy -2.493138 1.09626) (xy -2.493191 0.983287) (xy -2.493235 0.862801) (xy -2.49327 0.734563)
    (xy -2.493296 0.59833) (xy -2.493315 0.453863) (xy -2.493327 0.300922) (xy -2.493334 0.139265) (xy -2.493336 0.002288)
    (xy -2.493339 -0.166415) (xy -2.493348 -0.326215) (xy -2.493359 -0.477359) (xy -2.493369 -0.620093) (xy -2.493376 -0.754665)
    (xy -2.493376 -0.881321) (xy -2.493366 -1.000308) (xy -2.493342 -1.111874) (xy -2.493304 -1.216264) (xy -2.493246 -1.313727)
    (xy -2.493166 -1.404507) (xy -2.493061 -1.488854) (xy -2.492929 -1.567012) (xy -2.492765 -1.63923) (xy -2.492567 -1.705753)
    (xy -2.492333 -1.76683) (xy -2.492058 -1.822706) (xy -2.49174 -1.873629) (xy -2.491376 -1.919845) (xy -2.490963 -1.961601)
    (xy -2.490498 -1.999145) (xy -2.489978 -2.032722) (xy -2.4894 -2.06258) (xy -2.48876 -2.088965) (xy -2.488057 -2.112126)
    (xy -2.487286 -2.132307) (xy -2.486445 -2.149756) (xy -2.48553 -2.164721) (xy -2.48454 -2.177447) (xy -2.48347 -2.188182)
    (xy -2.482317 -2.197173) (xy -2.48108 -2.204666) (xy -2.479754 -2.210908) (xy -2.478337 -2.216146) (xy -2.476825 -2.220627)
    (xy -2.475216 -2.224598) (xy -2.473507 -2.228305) (xy -2.471694 -2.231996) (xy -2.469774 -2.235917) (xy -2.467746 -2.240315)
    (xy -2.465853 -2.244813) (xy -2.440199 -2.296834) (xy -2.40707 -2.344471) (xy -2.367401 -2.386939) (xy -2.322129 -2.423451)
    (xy -2.272191 -2.453223) (xy -2.218524 -2.475467) (xy -2.177839 -2.486437) (xy -2.174521 -2.486979) (xy -2.169703 -2.487493)
    (xy -2.163144 -2.487979) (xy -2.154604 -2.488437) (xy -2.143842 -2.48887) (xy -2.130618 -2.489276) (xy -2.114691 -2.489658)
    (xy -2.095821 -2.490015) (xy -2.073768 -2.49035) (xy -2.048291 -2.490661) (xy -2.019148 -2.490951) (xy -1.986101 -2.49122)
    (xy -1.948908 -2.491468) (xy -1.907329 -2.491696) (xy -1.861123 -2.491906) (xy -1.810049 -2.492098) (xy -1.753869 -2.492273)
    (xy -1.69234 -2.492431) (xy -1.625222 -2.492573) (xy -1.552275 -2.4927) (xy -1.473258 -2.492813) (xy -1.387931 -2.492913)
    (xy -1.296054 -2.493) (xy -1.197385 -2.493075) (xy -1.091685 -2.493138) (xy -0.978712 -2.493191) (xy -0.858226 -2.493235)
    (xy -0.729987 -2.49327) (xy -0.593755 -2.493296) (xy -0.449288 -2.493315) (xy -0.296347 -2.493327) (xy -0.13469 -2.493334)
    (xy 0.002288 -2.493336))
   (stroke (width 0) (type solid)) (fill solid) (layer "F.Cu")))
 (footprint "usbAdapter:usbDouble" (layer "F.Cu") (at 145.034 89.916)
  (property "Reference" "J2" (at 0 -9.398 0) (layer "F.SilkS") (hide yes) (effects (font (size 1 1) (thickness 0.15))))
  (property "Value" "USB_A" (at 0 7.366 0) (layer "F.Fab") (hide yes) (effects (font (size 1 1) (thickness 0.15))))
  (fp_rect (start -12.7 -9.271) (end 12.7 4.191) (stroke (width 0.1) (type default)) (fill none) (layer "F.SilkS"))
  (pad "1" thru_hole circle (at -10.16 2.54) (size 2 2) (drill 0.9) (layers "*.Cu" "*.Mask") (remove_unused_layers no) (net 1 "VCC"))
  (pad "2" thru_hole circle (at -10.16 0) (size 2 2) (drill 0.9) (layers "*.Cu" "*.Mask") (remove_unused_layers no) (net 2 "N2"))
  (pad "3" thru_hole circle (at -10.16 -2.54) (size 2 2) (drill 0.9) (layers "*.Cu" "*.Mask") (remove_unused_layers no) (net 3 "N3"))
  (pad "4" thru_hole circle (at -10.16 -5.08) (size 2 2) (drill 0.9) (layers "*.Cu" "*.Mask") (remove_unused_layers no) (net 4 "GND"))
  (pad "5" thru_hole circle (at -10.16 -7.62) (size 2 2) (drill 0.9) (layers "*.Cu" "*.Mask") (remove_unused_layers no) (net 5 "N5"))
  (pad "6" thru_hole circle (at 10.16 2.54) (size 2 2) (drill 0.9) (layers "*.Cu" "*.Mask") (remove_unused_layers no) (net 1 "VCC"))
  (pad "7" thru_hole circle (at 10.16 0) (size 2 2) (drill 0.9) (layers "*.Cu" "*.Mask") (remove_unused_layers no) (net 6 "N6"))
  (pad "8" thru_hole circle (at 10.16 -2.54) (size 2 2) (drill 0.9) (layers "*.Cu" "*.Mask") (remove_unused_layers no) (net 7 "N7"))
  (pad "9" thru_hole circle (at 10.16 -5.08) (size 2 2) (drill 0.9) (layers "*.Cu" "*.Mask") (remove_unused_layers no) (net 4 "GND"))
  (pad "10" thru_hole circle (at 10.16 -7.62) (size 2 2) (drill 0.9) (layers "*.Cu" "*.Mask") (remove_unused_layers no) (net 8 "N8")))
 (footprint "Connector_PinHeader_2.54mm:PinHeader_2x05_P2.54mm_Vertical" (layer "F.Cu") (at 169.926 84.582)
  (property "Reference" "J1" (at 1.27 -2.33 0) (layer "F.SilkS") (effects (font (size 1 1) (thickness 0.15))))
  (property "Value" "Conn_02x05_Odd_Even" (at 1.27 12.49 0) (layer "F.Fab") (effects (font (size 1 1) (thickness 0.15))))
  (fp_line (start -1.33 -1.33) (end 0 -1.33) (stroke (width 0.12) (type solid)) (layer "F.SilkS"))
  (fp_line (start -1.33 0) (end -1.33 -1.33) (stroke (width 0.12) (type solid)) (layer "F.SilkS"))
  (fp_line (start -1.33 1.27) (end -1.33 11.49) (stroke (width 0.12) (type solid)) (layer "F.SilkS"))
  (fp_line (start -1.33 1.27) (end 1.27 1.27) (stroke (width 0.12) (type solid)) (layer "F.SilkS"))
  (fp_line (start -1.33 11.49) (end 3.87 11.49) (stroke (width 0.12) (type solid)) (layer "F.SilkS"))
  (fp_line (start 1.27 -1.33) (end 3.87 -1.33) (stroke (width 0.12) (type solid)) (layer "F.SilkS"))
  (fp_line (start 1.27 1.27) (end 1.27 -1.33) (stroke (width 0.12) (type solid)) (layer "F.SilkS"))
  (fp_line (start 3.87 -1.33) (end 3.87 11.49) (stroke (width 0.12) (type solid)) (layer "F.SilkS"))
  (pad "1" thru_hole rect (at 0 0) (size 1.7 1.7) (drill 1) (layers "*.Cu" "*.Mask") (remove_unused_layers no) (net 1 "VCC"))
  (pad "2" thru_hole oval (at 2.54 0) (size 1.7 1.7) (drill 1) (layers "*.Cu" "*.Mask") (remove_unused_layers no) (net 1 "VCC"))
  (pad "3" thru_hole oval (at 0 2.54) (size 1.7 1.7) (drill 1) (layers "*.Cu" "*.Mask") (remove_unused_layers no) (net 7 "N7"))
  (pad "4" thru_hole oval (at 2.54 2.54) (size 1.7 1.7) (drill 1) (layers "*.Cu" "*.Mask") (remove_unused_layers no) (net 2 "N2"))
  (pad "5" thru_hole oval (at 0 5.08) (size 1.7 1.7) (drill 1) (layers "*.Cu" "*.Mask") (remove_unused_layers no) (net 6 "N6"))
  (pad "6" thru_hole oval (at 2.54 5.08) (size 1.7 1.7) (drill 1) (layers "*.Cu" "*.Mask") (remove_unused_layers no) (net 3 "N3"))
  (pad "7" thru_hole oval (at 0 7.62) (size 1.7 1.7) (drill 1) (layers "*.Cu" "*.Mask") (remove_unused_layers no) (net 4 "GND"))
  (pad "8" thru_hole oval (at 2.54 7.62) (size 1.7 1.7) (drill 1) (layers "*.Cu" "*.Mask") (remove_unused_layers no) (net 4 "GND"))
  (pad "9" thru_hole oval (at 0 10.16) (size 1.7 1.7) (drill 1) (layers "*.Cu" "*.Mask") (remove_unused_layers no) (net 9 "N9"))
  (pad "10" thru_hole oval (at 2.54 10.16) (size 1.7 1.7) (drill 1) (layers "*.Cu" "*.Mask") (remove_unused_layers no) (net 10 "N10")))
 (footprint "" (layer "F.Cu") (at 161.036 92.456)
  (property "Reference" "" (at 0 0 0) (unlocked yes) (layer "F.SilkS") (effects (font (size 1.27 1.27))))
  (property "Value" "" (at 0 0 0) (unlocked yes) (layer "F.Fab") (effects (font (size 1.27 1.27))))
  (pad "6" thru_hole circle (at 0 0) (size 2 2) (drill 0.9) (layers "*.Cu" "*.Mask") (remove_unused_layers no) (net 1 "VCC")))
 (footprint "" (layer "F.Cu") (at 165.608 92.456)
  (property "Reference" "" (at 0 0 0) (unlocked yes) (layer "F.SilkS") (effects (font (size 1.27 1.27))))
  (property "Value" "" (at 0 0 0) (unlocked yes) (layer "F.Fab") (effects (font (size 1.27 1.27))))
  (pad "9" thru_hole circle (at 0 0) (size 2 2) (drill 0.9) (layers "*.Cu" "*.Mask") (remove_unused_layers no) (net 4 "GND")))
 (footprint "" (layer "F.Cu") (at 165.608 84.963)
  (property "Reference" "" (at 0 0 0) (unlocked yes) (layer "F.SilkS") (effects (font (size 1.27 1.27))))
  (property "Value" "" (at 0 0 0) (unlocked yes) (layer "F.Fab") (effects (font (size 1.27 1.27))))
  (pad "9" thru_hole circle (at 0 0) (size 2 2) (drill 0.9) (layers "*.Cu" "*.Mask") (remove_unused_layers no) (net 4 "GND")))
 (gr_rect (start 127.127 75.946) (end 183.388 102.362) (stroke (width 0.05) (type default)) (fill none) (layer "Edge.Cuts"))
 (segment (start 155.321 78.74) (end 131.191 78.74) (width 0.9) (layer "F.Cu") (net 1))
 (segment (start 161.036 82.042) (end 161.036 78.867) (width 0.9) (layer "F.Cu") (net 1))
 (segment (start 135.001 92.456) (end 129.413 92.456) (width 0.9) (layer "F.Cu") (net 1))
 (segment (start 129.413 80.518) (end 131.191 78.74) (width 0.9) (layer "F.Cu") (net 1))
 (segment (start 169.799 84.582) (end 169.799 79.756) (width 0.9) (layer "F.Cu") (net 1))
 (segment (start 161.036 78.867) (end 161.163 78.74) (width 0.9) (layer "F.Cu") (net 1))
 (segment (start 129.413 92.456) (end 129.413 80.518) (width 0.9) (layer "F.Cu") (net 1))
 (segment (start 169.799 79.756) (end 168.783 78.74) (width 0.9) (layer "F.Cu") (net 1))
 (segment (start 172.339 84.582) (end 169.799 84.582) (width 0.9) (layer "F.Cu") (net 1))
 (segment (start 168.783 78.74) (end 161.163 78.74) (width 0.9) (layer "F.Cu") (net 1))
 (segment (start 161.163 78.74) (end 155.321 78.74) (width 0.9) (layer "F.Cu") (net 1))
 (segment (start 155.194 92.456) (end 161.036 92.456) (width 0.9) (layer "F.Cu") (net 1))
 (segment (start 161.036 92.456) (end 161.036 82.042) (width 0.9) (layer "B.Cu") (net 1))
 (segment (start 169.799 92.202) (end 165.862 92.202) (width 0.9) (layer "F.Cu") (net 4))
 (segment (start 169.799 92.202) (end 172.339 92.202) (width 0.9) (layer "F.Cu") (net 4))
 (segment (start 134.874 84.836) (end 155.194 84.836) (width 0.9) (layer "F.Cu") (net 4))
 (segment (start 165.862 92.202) (end 165.608 92.456) (width 0.9) (layer "F.Cu") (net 4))
 (segment (start 165.608 84.963) (end 155.321 84.963) (width 0.9) (layer "F.Cu") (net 4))
 (segment (start 155.321 84.963) (end 155.194 84.836) (width 0.9) (layer "F.Cu") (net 4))
 (segment (start 165.608 84.963) (end 165.608 92.456) (width 0.9) (layer "B.Cu") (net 4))
 (segment (start 169.545 89.916) (end 155.194 89.916) (width 0.9) (layer "F.Cu") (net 6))
 (segment (start 169.799 89.662) (end 169.545 89.916) (width 0.9) (layer "F.Cu") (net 6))
 (segment (start 169.799 87.122) (end 169.545 87.376) (width 0.9) (layer "F.Cu") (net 7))
 (segment (start 169.545 87.376) (end 155.194 87.376) (width 0.9) (layer "F.Cu") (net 7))
 (segment (start 138.562584 87.376) (end 135.001 87.376) (width 0.9) (layer "F.Cu") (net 3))
 (segment (start 177.695 98.022) (end 140.694 98.022) (width 0.9) (layer "F.Cu") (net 3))
 (segment (start 179.048 89.662) (end 179.048 96.669) (width 0.9) (layer "F.Cu") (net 3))
 (segment (start 179.048 96.669) (end 177.695 98.022) (width 0.9) (layer "F.Cu") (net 3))
 (segment (start 172.339 89.662) (end 179.048 89.662) (width 0.9) (layer "F.Cu") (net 3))
 (segment (start 140.589 89.402416) (end 138.562584 87.376) (width 0.9) (layer "F.Cu") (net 3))
 (segment (start 140.694 98.022) (end 140.589 97.917) (width 0.9) (layer "F.Cu") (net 3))
 (segment (start 140.589 97.917) (end 140.589 89.402416) (width 0.9) (layer "F.Cu") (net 3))
 (segment (start 180.848 87.757) (end 180.848 98.044) (width 0.9) (layer "F.Cu") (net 2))
 (segment (start 179.07 99.822) (end 138.557 99.822) (width 0.9) (layer "F.Cu") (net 2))
 (segment (start 172.339 87.122) (end 180.213 87.122) (width 0.9) (layer "F.Cu") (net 2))
 (segment (start 138.557 89.916) (end 135.001 89.916) (width 0.9) (layer "F.Cu") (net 2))
 (segment (start 138.557 99.822) (end 138.557 89.916) (width 0.9) (layer "F.Cu") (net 2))
 (segment (start 180.848 98.044) (end 179.07 99.822) (width 0.9) (layer "F.Cu") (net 2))
 (segment (start 180.213 87.122) (end 180.848 87.757) (width 0.9) (layer "F.Cu") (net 2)))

